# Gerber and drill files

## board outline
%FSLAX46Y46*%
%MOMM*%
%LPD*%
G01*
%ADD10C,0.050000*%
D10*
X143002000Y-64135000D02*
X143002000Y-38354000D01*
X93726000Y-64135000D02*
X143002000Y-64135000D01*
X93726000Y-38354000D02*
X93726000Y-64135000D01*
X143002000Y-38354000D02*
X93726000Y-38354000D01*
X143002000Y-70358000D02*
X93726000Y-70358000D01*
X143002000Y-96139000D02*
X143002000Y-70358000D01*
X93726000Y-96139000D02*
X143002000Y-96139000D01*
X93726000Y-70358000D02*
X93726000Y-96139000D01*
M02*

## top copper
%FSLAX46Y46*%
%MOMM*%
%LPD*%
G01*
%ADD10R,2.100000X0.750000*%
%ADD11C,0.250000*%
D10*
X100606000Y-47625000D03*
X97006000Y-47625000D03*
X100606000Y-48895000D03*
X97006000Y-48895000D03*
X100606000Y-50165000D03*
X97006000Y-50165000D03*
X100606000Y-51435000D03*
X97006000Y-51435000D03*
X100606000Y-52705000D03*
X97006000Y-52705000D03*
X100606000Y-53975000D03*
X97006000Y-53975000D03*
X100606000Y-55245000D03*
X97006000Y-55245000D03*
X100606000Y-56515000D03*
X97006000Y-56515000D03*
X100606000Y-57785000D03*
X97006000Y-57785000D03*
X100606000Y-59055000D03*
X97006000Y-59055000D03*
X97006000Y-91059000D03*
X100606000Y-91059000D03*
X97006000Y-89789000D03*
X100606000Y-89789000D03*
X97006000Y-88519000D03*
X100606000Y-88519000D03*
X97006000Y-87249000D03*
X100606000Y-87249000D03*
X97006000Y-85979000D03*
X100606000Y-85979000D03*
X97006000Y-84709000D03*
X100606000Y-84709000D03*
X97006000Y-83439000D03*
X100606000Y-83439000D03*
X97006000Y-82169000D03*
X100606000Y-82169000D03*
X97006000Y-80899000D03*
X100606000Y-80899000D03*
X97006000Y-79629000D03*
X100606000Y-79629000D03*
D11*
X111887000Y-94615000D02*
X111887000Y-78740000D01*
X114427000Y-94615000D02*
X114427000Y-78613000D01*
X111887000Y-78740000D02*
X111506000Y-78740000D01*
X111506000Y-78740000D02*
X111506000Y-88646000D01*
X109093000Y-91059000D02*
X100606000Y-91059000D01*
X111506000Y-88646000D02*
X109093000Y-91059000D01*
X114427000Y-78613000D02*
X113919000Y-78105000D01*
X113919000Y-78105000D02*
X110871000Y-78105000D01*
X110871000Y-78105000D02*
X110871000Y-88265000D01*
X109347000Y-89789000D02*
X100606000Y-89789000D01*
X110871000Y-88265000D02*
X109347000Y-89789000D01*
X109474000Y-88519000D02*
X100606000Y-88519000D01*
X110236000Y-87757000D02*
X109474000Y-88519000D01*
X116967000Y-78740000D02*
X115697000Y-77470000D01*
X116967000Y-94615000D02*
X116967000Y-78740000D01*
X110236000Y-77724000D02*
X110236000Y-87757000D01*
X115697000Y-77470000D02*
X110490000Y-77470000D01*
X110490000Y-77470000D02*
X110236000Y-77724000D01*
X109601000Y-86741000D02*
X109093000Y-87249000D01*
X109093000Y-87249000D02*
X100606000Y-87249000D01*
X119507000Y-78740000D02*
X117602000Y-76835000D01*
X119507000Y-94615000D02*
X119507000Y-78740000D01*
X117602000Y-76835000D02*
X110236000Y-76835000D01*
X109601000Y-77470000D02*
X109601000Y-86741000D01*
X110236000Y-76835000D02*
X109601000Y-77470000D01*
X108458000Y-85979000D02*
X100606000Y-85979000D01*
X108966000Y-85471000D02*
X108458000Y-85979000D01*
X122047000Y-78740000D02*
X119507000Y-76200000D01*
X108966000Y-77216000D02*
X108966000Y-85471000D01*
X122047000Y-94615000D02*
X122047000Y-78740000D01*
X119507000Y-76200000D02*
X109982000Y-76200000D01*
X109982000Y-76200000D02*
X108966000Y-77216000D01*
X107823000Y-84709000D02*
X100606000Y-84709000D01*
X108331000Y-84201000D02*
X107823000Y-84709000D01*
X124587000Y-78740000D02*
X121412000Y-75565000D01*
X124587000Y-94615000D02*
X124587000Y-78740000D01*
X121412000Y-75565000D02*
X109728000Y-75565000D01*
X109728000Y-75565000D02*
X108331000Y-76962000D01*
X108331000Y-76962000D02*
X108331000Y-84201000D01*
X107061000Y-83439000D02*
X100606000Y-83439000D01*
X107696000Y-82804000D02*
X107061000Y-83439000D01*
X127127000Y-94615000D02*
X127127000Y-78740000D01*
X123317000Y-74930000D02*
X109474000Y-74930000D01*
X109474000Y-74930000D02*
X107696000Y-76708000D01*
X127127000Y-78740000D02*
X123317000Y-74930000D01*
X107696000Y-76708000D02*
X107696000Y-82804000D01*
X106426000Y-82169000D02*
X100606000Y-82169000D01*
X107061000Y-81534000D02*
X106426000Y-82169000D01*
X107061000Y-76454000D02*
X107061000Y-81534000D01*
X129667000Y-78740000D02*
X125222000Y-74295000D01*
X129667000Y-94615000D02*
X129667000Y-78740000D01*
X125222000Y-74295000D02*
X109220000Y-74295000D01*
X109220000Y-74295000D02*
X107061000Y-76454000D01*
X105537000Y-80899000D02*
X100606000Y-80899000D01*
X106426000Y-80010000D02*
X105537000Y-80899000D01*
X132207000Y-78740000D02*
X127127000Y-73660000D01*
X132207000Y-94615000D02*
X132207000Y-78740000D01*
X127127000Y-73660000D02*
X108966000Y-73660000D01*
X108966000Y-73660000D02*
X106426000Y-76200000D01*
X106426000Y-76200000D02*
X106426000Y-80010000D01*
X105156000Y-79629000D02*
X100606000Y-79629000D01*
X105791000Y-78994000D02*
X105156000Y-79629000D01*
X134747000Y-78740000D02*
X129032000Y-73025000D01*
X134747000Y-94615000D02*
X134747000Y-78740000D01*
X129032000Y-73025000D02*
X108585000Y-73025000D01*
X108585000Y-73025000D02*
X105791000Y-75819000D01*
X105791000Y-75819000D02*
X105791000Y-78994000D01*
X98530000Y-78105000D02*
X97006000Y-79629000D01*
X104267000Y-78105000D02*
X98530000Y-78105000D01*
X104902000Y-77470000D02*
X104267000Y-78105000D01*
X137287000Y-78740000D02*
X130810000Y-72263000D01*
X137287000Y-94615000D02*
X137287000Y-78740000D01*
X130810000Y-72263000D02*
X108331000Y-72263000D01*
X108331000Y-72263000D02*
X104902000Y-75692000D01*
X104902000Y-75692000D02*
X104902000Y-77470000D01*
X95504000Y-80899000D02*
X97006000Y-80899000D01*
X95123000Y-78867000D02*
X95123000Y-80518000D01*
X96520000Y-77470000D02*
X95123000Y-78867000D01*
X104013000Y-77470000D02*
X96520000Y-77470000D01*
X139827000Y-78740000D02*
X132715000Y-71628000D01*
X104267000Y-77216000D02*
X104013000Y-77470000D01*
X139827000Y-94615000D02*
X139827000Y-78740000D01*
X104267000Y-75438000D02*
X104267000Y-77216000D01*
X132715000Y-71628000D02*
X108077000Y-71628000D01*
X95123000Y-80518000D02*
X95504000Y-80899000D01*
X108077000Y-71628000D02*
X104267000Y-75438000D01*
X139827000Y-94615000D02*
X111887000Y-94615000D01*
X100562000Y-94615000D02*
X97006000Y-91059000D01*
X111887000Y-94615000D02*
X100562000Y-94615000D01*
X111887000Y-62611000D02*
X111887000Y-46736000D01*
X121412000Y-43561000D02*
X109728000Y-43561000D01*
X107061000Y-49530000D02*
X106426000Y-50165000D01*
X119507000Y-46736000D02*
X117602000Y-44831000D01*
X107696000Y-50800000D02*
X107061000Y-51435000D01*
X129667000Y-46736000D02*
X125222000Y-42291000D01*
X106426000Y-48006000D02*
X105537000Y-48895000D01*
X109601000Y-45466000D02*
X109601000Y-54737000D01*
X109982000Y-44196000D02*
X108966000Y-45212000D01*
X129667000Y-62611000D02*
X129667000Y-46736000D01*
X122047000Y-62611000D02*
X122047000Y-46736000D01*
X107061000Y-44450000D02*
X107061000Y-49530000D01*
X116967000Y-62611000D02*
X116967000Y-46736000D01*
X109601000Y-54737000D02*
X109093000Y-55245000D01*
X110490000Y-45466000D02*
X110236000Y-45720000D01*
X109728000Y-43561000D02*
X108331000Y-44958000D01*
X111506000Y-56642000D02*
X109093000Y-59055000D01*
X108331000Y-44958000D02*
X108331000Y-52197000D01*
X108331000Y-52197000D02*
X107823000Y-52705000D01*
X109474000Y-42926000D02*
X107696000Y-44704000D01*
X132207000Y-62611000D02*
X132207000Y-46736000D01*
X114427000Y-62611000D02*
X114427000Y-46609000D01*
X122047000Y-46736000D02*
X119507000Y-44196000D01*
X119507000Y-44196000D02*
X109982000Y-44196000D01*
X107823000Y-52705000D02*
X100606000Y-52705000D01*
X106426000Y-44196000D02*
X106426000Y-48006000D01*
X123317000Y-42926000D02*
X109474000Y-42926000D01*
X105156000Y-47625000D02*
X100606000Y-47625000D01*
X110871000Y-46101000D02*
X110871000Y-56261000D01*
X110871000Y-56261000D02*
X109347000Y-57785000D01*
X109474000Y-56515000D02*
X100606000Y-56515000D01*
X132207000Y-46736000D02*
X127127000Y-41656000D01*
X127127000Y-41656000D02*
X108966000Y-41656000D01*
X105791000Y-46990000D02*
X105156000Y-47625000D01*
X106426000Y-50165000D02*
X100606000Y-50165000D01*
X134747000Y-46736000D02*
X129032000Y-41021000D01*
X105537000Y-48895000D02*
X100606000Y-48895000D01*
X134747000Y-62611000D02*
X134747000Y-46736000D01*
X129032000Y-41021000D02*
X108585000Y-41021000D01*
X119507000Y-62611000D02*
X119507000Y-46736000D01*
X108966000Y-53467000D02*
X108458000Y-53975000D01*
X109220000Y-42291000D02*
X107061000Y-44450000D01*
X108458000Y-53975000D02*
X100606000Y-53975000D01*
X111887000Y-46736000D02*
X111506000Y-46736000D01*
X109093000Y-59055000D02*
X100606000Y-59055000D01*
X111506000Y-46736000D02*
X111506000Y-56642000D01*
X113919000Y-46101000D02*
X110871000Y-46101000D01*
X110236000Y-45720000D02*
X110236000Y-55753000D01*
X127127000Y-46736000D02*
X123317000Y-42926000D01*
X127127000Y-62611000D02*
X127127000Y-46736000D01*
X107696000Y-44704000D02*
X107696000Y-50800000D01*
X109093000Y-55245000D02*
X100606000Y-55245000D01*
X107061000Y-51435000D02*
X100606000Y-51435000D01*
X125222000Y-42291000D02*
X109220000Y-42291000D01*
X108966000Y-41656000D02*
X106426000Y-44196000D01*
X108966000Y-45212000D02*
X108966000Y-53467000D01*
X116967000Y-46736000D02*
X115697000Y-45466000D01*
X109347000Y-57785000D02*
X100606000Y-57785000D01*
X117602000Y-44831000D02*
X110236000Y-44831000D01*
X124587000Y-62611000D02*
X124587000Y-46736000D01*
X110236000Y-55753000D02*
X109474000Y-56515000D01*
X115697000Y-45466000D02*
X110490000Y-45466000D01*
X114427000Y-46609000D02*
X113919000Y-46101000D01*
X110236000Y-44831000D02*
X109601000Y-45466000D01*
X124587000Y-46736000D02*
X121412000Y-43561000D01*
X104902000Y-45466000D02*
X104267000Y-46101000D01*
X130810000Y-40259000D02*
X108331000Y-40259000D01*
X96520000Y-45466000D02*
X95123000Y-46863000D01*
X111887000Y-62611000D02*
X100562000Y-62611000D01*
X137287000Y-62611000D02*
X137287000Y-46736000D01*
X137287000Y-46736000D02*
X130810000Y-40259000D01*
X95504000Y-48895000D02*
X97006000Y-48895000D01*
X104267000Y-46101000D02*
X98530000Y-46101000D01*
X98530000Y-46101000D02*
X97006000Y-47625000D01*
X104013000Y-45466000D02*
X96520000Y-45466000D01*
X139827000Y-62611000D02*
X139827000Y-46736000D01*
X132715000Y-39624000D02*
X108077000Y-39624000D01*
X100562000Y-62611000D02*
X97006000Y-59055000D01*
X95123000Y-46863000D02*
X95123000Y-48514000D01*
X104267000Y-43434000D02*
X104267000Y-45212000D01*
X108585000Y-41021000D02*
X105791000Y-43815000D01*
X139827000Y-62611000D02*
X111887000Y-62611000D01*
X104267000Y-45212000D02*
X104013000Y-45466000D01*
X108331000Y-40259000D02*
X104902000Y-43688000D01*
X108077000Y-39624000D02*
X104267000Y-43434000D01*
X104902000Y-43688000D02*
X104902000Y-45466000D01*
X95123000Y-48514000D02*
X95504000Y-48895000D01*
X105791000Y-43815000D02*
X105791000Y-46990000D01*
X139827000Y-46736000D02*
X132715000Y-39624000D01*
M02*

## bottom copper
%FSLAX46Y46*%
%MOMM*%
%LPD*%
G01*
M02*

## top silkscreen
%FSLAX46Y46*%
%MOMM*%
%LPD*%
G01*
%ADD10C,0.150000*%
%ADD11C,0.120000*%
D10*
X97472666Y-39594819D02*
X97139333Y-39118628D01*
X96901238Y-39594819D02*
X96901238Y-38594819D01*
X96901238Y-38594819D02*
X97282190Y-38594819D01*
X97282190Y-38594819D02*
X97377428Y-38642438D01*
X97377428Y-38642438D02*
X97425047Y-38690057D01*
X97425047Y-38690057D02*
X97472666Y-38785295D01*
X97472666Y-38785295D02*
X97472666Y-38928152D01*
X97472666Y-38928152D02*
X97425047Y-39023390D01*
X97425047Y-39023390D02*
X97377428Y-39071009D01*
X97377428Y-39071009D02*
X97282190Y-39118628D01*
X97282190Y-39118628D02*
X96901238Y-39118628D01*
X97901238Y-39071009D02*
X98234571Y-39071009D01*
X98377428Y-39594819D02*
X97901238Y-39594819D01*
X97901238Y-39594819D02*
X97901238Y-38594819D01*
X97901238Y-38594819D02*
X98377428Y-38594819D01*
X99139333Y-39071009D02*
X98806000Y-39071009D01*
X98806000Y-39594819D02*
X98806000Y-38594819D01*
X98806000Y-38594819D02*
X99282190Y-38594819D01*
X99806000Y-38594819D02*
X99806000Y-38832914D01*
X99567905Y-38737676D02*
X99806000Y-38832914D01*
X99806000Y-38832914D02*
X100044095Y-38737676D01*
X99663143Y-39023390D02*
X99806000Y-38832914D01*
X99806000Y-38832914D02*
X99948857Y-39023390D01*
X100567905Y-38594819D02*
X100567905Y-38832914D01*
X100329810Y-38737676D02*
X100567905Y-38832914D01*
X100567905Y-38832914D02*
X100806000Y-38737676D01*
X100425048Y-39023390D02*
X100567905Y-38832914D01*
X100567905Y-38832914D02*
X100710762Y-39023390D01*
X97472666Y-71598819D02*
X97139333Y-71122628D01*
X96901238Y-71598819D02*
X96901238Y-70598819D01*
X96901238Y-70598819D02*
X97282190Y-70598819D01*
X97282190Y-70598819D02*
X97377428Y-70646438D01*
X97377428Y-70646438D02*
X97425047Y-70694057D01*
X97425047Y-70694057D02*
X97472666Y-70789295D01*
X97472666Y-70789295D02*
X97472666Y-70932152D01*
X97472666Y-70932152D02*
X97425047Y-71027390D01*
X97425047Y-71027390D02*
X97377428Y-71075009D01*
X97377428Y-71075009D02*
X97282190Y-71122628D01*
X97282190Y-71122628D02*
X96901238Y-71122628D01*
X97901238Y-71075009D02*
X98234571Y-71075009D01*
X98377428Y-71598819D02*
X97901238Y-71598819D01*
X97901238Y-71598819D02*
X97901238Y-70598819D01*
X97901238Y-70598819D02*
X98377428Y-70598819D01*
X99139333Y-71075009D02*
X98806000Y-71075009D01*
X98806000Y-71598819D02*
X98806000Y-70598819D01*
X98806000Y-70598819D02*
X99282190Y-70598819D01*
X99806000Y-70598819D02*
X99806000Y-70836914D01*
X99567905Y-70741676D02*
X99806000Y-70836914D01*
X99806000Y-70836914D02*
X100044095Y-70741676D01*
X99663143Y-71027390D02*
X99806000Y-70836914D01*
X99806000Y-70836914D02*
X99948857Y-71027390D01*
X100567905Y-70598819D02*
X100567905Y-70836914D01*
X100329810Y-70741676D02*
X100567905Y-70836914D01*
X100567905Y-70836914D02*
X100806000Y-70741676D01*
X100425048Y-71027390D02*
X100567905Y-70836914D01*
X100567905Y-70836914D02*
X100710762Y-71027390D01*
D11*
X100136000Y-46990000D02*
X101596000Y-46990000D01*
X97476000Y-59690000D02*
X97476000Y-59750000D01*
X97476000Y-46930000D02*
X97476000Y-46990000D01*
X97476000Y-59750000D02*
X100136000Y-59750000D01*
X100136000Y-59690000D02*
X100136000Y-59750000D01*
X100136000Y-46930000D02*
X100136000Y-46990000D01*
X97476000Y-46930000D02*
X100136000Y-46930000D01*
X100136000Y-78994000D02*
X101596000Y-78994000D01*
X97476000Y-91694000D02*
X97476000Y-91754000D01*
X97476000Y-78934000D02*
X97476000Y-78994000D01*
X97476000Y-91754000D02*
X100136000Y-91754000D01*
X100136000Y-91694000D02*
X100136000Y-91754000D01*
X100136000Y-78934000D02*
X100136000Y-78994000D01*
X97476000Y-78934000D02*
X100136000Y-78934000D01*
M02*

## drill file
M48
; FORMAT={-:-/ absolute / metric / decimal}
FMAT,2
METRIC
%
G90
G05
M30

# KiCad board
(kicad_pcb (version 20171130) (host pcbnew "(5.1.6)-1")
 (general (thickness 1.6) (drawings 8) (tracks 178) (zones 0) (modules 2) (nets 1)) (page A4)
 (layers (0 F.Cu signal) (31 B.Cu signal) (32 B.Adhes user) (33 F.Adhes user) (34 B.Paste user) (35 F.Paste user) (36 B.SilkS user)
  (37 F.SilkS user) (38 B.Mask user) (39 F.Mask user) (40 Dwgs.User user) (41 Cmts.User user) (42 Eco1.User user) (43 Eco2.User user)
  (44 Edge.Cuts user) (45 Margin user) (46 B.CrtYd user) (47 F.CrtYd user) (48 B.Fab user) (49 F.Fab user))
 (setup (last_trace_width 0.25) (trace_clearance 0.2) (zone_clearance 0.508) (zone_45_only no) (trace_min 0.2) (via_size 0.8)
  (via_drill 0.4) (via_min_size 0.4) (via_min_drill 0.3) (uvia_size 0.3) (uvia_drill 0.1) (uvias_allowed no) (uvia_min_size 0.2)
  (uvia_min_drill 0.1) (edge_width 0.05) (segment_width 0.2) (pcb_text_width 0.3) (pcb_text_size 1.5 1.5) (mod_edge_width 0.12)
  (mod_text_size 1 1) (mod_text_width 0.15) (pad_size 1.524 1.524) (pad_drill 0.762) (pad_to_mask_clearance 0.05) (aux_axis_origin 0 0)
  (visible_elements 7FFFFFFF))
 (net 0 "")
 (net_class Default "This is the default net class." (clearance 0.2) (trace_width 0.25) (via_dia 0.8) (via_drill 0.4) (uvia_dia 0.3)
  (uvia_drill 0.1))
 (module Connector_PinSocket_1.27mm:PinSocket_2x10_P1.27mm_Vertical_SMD (layer F.Cu) (at 98.806 53.34)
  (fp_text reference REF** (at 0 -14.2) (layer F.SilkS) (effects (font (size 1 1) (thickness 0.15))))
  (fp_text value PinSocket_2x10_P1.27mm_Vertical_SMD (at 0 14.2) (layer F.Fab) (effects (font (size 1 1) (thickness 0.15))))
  (fp_line (start 1.33 -6.35) (end 2.79 -6.35) (layer F.SilkS) (width 0.12))
  (fp_line (start -1.33 6.35) (end -1.33 6.41) (layer F.SilkS) (width 0.12))
  (fp_line (start -1.33 -6.41) (end -1.33 -6.35) (layer F.SilkS) (width 0.12))
  (fp_line (start -1.33 6.41) (end 1.33 6.41) (layer F.SilkS) (width 0.12))
  (fp_line (start 1.33 6.35) (end 1.33 6.41) (layer F.SilkS) (width 0.12))
  (fp_line (start 1.33 -6.41) (end 1.33 -6.35) (layer F.SilkS) (width 0.12))
  (fp_line (start -1.33 -6.41) (end 1.33 -6.41) (layer F.SilkS) (width 0.12))
  (pad 1 smd rect (at 1.8 -5.715) (size 2.1 0.75) (layers F.Cu F.Paste F.Mask))
  (pad 2 smd rect (at -1.8 -5.715) (size 2.1 0.75) (layers F.Cu F.Paste F.Mask))
  (pad 3 smd rect (at 1.8 -4.445) (size 2.1 0.75) (layers F.Cu F.Paste F.Mask))
  (pad 4 smd rect (at -1.8 -4.445) (size 2.1 0.75) (layers F.Cu F.Paste F.Mask))
  (pad 5 smd rect (at 1.8 -3.175) (size 2.1 0.75) (layers F.Cu F.Paste F.Mask))
  (pad 6 smd rect (at -1.8 -3.175) (size 2.1 0.75) (layers F.Cu F.Paste F.Mask))
  (pad 7 smd rect (at 1.8 -1.905) (size 2.1 0.75) (layers F.Cu F.Paste F.Mask))
  (pad 8 smd rect (at -1.8 -1.905) (size 2.1 0.75) (layers F.Cu F.Paste F.Mask))
  (pad 9 smd rect (at 1.8 -0.635) (size 2.1 0.75) (layers F.Cu F.Paste F.Mask))
  (pad 10 smd rect (at -1.8 -0.635) (size 2.1 0.75) (layers F.Cu F.Paste F.Mask))
  (pad 11 smd rect (at 1.8 0.635) (size 2.1 0.75) (layers F.Cu F.Paste F.Mask))
  (pad 12 smd rect (at -1.8 0.635) (size 2.1 0.75) (layers F.Cu F.Paste F.Mask))
  (pad 13 smd rect (at 1.8 1.905) (size 2.1 0.75) (layers F.Cu F.Paste F.Mask))
  (pad 14 smd rect (at -1.8 1.905) (size 2.1 0.75) (layers F.Cu F.Paste F.Mask))
  (pad 15 smd rect (at 1.8 3.175) (size 2.1 0.75) (layers F.Cu F.Paste F.Mask))
  (pad 16 smd rect (at -1.8 3.175) (size 2.1 0.75) (layers F.Cu F.Paste F.Mask))
  (pad 17 smd rect (at 1.8 4.445) (size 2.1 0.75) (layers F.Cu F.Paste F.Mask))
  (pad 18 smd rect (at -1.8 4.445) (size 2.1 0.75) (layers F.Cu F.Paste F.Mask))
  (pad 19 smd rect (at 1.8 5.715) (size 2.1 0.75) (layers F.Cu F.Paste F.Mask))
  (pad 20 smd rect (at -1.8 5.715) (size 2.1 0.75) (layers F.Cu F.Paste F.Mask)))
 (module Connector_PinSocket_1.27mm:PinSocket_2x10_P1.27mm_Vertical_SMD (layer F.Cu) (at 98.806 85.344)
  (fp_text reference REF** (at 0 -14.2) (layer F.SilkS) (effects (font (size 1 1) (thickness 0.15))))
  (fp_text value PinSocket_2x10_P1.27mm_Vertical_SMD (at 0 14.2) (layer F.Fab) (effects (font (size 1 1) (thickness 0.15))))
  (fp_line (start 1.33 -6.35) (end 2.79 -6.35) (layer F.SilkS) (width 0.12))
  (fp_line (start -1.33 6.35) (end -1.33 6.41) (layer F.SilkS) (width 0.12))
  (fp_line (start -1.33 -6.41) (end -1.33 -6.35) (layer F.SilkS) (width 0.12))
  (fp_line (start -1.33 6.41) (end 1.33 6.41) (layer F.SilkS) (width 0.12))
  (fp_line (start 1.33 6.35) (end 1.33 6.41) (layer F.SilkS) (width 0.12))
  (fp_line (start 1.33 -6.41) (end 1.33 -6.35) (layer F.SilkS) (width 0.12))
  (fp_line (start -1.33 -6.41) (end 1.33 -6.41) (layer F.SilkS) (width 0.12))
  (pad 20 smd rect (at -1.8 5.715) (size 2.1 0.75) (layers F.Cu F.Paste F.Mask))
  (pad 19 smd rect (at 1.8 5.715) (size 2.1 0.75) (layers F.Cu F.Paste F.Mask))
  (pad 18 smd rect (at -1.8 4.445) (size 2.1 0.75) (layers F.Cu F.Paste F.Mask))
  (pad 17 smd rect (at 1.8 4.445) (size 2.1 0.75) (layers F.Cu F.Paste F.Mask))
  (pad 16 smd rect (at -1.8 3.175) (size 2.1 0.75) (layers F.Cu F.Paste F.Mask))
  (pad 15 smd rect (at 1.8 3.175) (size 2.1 0.75) (layers F.Cu F.Paste F.Mask))
  (pad 14 smd rect (at -1.8 1.905) (size 2.1 0.75) (layers F.Cu F.Paste F.Mask))
  (pad 13 smd rect (at 1.8 1.905) (size 2.1 0.75) (layers F.Cu F.Paste F.Mask))
  (pad 12 smd rect (at -1.8 0.635) (size 2.1 0.75) (layers F.Cu F.Paste F.Mask))
  (pad 11 smd rect (at 1.8 0.635) (size 2.1 0.75) (layers F.Cu F.Paste F.Mask))
  (pad 10 smd rect (at -1.8 -0.635) (size 2.1 0.75) (layers F.Cu F.Paste F.Mask))
  (pad 9 smd rect (at 1.8 -0.635) (size 2.1 0.75) (layers F.Cu F.Paste F.Mask))
  (pad 8 smd rect (at -1.8 -1.905) (size 2.1 0.75) (layers F.Cu F.Paste F.Mask))
  (pad 7 smd rect (at 1.8 -1.905) (size 2.1 0.75) (layers F.Cu F.Paste F.Mask))
  (pad 6 smd rect (at -1.8 -3.175) (size 2.1 0.75) (layers F.Cu F.Paste F.Mask))
  (pad 5 smd rect (at 1.8 -3.175) (size 2.1 0.75) (layers F.Cu F.Paste F.Mask))
  (pad 4 smd rect (at -1.8 -4.445) (size 2.1 0.75) (layers F.Cu F.Paste F.Mask))
  (pad 3 smd rect (at 1.8 -4.445) (size 2.1 0.75) (layers F.Cu F.Paste F.Mask))
  (pad 2 smd rect (at -1.8 -5.715) (size 2.1 0.75) (layers F.Cu F.Paste F.Mask))
  (pad 1 smd rect (at 1.8 -5.715) (size 2.1 0.75) (layers F.Cu F.Paste F.Mask)))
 (gr_line (start 143.002 64.135) (end 143.002 38.354) (layer Edge.Cuts) (width 0.05))
 (gr_line (start 93.726 64.135) (end 143.002 64.135) (layer Edge.Cuts) (width 0.05))
 (gr_line (start 93.726 38.354) (end 93.726 64.135) (layer Edge.Cuts) (width 0.05))
 (gr_line (start 143.002 38.354) (end 93.726 38.354) (layer Edge.Cuts) (width 0.05))
 (gr_line (start 143.002 70.358) (end 93.726 70.358) (layer Edge.Cuts) (width 0.05))
 (gr_line (start 143.002 96.139) (end 143.002 70.358) (layer Edge.Cuts) (width 0.05))
 (gr_line (start 93.726 96.139) (end 143.002 96.139) (layer Edge.Cuts) (width 0.05))
 (gr_line (start 93.726 70.358) (end 93.726 96.139) (layer Edge.Cuts) (width 0.05))
 (segment (start 111.887 94.615) (end 111.887 78.74) (width 0.25) (layer F.Cu) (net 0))
 (segment (start 114.427 94.615) (end 114.427 78.613) (width 0.25) (layer F.Cu) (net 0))
 (segment (start 111.887 78.74) (end 111.506 78.74) (width 0.25) (layer F.Cu) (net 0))
 (segment (start 111.506 78.74) (end 111.506 88.646) (width 0.25) (layer F.Cu) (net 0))
 (segment (start 109.093 91.059) (end 100.606 91.059) (width 0.25) (layer F.Cu) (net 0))
 (segment (start 111.506 88.646) (end 109.093 91.059) (width 0.25) (layer F.Cu) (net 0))
 (segment (start 114.427 78.613) (end 113.919 78.105) (width 0.25) (layer F.Cu) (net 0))
 (segment (start 113.919 78.105) (end 110.871 78.105) (width 0.25) (layer F.Cu) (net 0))
 (segment (start 110.871 78.105) (end 110.871 88.265) (width 0.25) (layer F.Cu) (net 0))
 (segment (start 109.347 89.789) (end 100.606 89.789) (width 0.25) (layer F.Cu) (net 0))
 (segment (start 110.871 88.265) (end 109.347 89.789) (width 0.25) (layer F.Cu) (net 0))
 (segment (start 109.474 88.519) (end 100.606 88.519) (width 0.25) (layer F.Cu) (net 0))
 (segment (start 110.236 87.757) (end 109.474 88.519) (width 0.25) (layer F.Cu) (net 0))
 (segment (start 116.967 78.74) (end 115.697 77.47) (width 0.25) (layer F.Cu) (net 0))
 (segment (start 116.967 94.615) (end 116.967 78.74) (width 0.25) (layer F.Cu) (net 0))
 (segment (start 110.236 77.724) (end 110.236 87.757) (width 0.25) (layer F.Cu) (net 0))
 (segment (start 115.697 77.47) (end 110.49 77.47) (width 0.25) (layer F.Cu) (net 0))
 (segment (start 110.49 77.47) (end 110.236 77.724) (width 0.25) (layer F.Cu) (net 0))
 (segment (start 109.601 86.741) (end 109.093 87.249) (width 0.25) (layer F.Cu) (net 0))
 (segment (start 109.093 87.249) (end 100.606 87.249) (width 0.25) (layer F.Cu) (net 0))
 (segment (start 119.507 78.74) (end 117.602 76.835) (width 0.25) (layer F.Cu) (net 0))
 (segment (start 119.507 94.615) (end 119.507 78.74) (width 0.25) (layer F.Cu) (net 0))
 (segment (start 117.602 76.835) (end 110.236 76.835) (width 0.25) (layer F.Cu) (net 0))
 (segment (start 109.601 77.47) (end 109.601 86.741) (width 0.25) (layer F.Cu) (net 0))
 (segment (start 110.236 76.835) (end 109.601 77.47) (width 0.25) (layer F.Cu) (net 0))
 (segment (start 108.458 85.979) (end 100.606 85.979) (width 0.25) (layer F.Cu) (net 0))
 (segment (start 108.966 85.471) (end 108.458 85.979) (width 0.25) (layer F.Cu) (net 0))
 (segment (start 122.047 78.74) (end 119.507 76.2) (width 0.25) (layer F.Cu) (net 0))
 (segment (start 108.966 77.216) (end 108.966 85.471) (width 0.25) (layer F.Cu) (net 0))
 (segment (start 122.047 94.615) (end 122.047 78.74) (width 0.25) (layer F.Cu) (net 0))
 (segment (start 119.507 76.2) (end 109.982 76.2) (width 0.25) (layer F.Cu) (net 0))
 (segment (start 109.982 76.2) (end 108.966 77.216) (width 0.25) (layer F.Cu) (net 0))
 (segment (start 107.823 84.709) (end 100.606 84.709) (width 0.25) (layer F.Cu) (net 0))
 (segment (start 108.331 84.201) (end 107.823 84.709) (width 0.25) (layer F.Cu) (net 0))
 (segment (start 124.587 78.74) (end 121.412 75.565) (width 0.25) (layer F.Cu) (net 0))
 (segment (start 124.587 94.615) (end 124.587 78.74) (width 0.25) (layer F.Cu) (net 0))
 (segment (start 121.412 75.565) (end 109.728 75.565) (width 0.25) (layer F.Cu) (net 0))
 (segment (start 109.728 75.565) (end 108.331 76.962) (width 0.25) (layer F.Cu) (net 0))
 (segment (start 108.331 76.962) (end 108.331 84.201) (width 0.25) (layer F.Cu) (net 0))
 (segment (start 107.061 83.439) (end 100.606 83.439) (width 0.25) (layer F.Cu) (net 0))
 (segment (start 107.696 82.804) (end 107.061 83.439) (width 0.25) (layer F.Cu) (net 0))
 (segment (start 127.127 94.615) (end 127.127 78.74) (width 0.25) (layer F.Cu) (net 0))
 (segment (start 123.317 74.93) (end 109.474 74.93) (width 0.25) (layer F.Cu) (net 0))
 (segment (start 109.474 74.93) (end 107.696 76.708) (width 0.25) (layer F.Cu) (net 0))
 (segment (start 127.127 78.74) (end 123.317 74.93) (width 0.25) (layer F.Cu) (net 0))
 (segment (start 107.696 76.708) (end 107.696 82.804) (width 0.25) (layer F.Cu) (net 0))
 (segment (start 106.426 82.169) (end 100.606 82.169) (width 0.25) (layer F.Cu) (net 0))
 (segment (start 107.061 81.534) (end 106.426 82.169) (width 0.25) (layer F.Cu) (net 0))
 (segment (start 107.061 76.454) (end 107.061 81.534) (width 0.25) (layer F.Cu) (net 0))
 (segment (start 129.667 78.74) (end 125.222 74.295) (width 0.25) (layer F.Cu) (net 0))
 (segment (start 129.667 94.615) (end 129.667 78.74) (width 0.25) (layer F.Cu) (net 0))
 (segment (start 125.222 74.295) (end 109.22 74.295) (width 0.25) (layer F.Cu) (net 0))
 (segment (start 109.22 74.295) (end 107.061 76.454) (width 0.25) (layer F.Cu) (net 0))
 (segment (start 105.537 80.899) (end 100.606 80.899) (width 0.25) (layer F.Cu) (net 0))
 (segment (start 106.426 80.01) (end 105.537 80.899) (width 0.25) (layer F.Cu) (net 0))
 (segment (start 132.207 78.74) (end 127.127 73.66) (width 0.25) (layer F.Cu) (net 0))
 (segment (start 132.207 94.615) (end 132.207 78.74) (width 0.25) (layer F.Cu) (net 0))
 (segment (start 127.127 73.66) (end 108.966 73.66) (width 0.25) (layer F.Cu) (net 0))
 (segment (start 108.966 73.66) (end 106.426 76.2) (width 0.25) (layer F.Cu) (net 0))
 (segment (start 106.426 76.2) (end 106.426 80.01) (width 0.25) (layer F.Cu) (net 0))
 (segment (start 105.156 79.629) (end 100.606 79.629) (width 0.25) (layer F.Cu) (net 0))
 (segment (start 105.791 78.994) (end 105.156 79.629) (width 0.25) (layer F.Cu) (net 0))
 (segment (start 134.747 78.74) (end 129.032 73.025) (width 0.25) (layer F.Cu) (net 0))
 (segment (start 134.747 94.615) (end 134.747 78.74) (width 0.25) (layer F.Cu) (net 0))
 (segment (start 129.032 73.025) (end 108.585 73.025) (width 0.25) (layer F.Cu) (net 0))
 (segment (start 108.585 73.025) (end 105.791 75.819) (width 0.25) (layer F.Cu) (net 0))
 (segment (start 105.791 75.819) (end 105.791 78.994) (width 0.25) (layer F.Cu) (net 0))
 (segment (start 98.53 78.105) (end 97.006 79.629) (width 0.25) (layer F.Cu) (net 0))
 (segment (start 104.267 78.105) (end 98.53 78.105) (width 0.25) (layer F.Cu) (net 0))
 (segment (start 104.902 77.47) (end 104.267 78.105) (width 0.25) (layer F.Cu) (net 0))
 (segment (start 137.287 78.74) (end 130.81 72.263) (width 0.25) (layer F.Cu) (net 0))
 (segment (start 137.287 94.615) (end 137.287 78.74) (width 0.25) (layer F.Cu) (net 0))
 (segment (start 130.81 72.263) (end 108.331 72.263) (width 0.25) (layer F.Cu) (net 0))
 (segment (start 108.331 72.263) (end 104.902 75.692) (width 0.25) (layer F.Cu) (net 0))
 (segment (start 104.902 75.692) (end 104.902 77.47) (width 0.25) (layer F.Cu) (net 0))
 (segment (start 95.504 80.899) (end 97.006 80.899) (width 0.25) (layer F.Cu) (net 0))
 (segment (start 95.123 78.867) (end 95.123 80.518) (width 0.25) (layer F.Cu) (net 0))
 (segment (start 96.52 77.47) (end 95.123 78.867) (width 0.25) (layer F.Cu) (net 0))
 (segment (start 104.013 77.47) (end 96.52 77.47) (width 0.25) (layer F.Cu) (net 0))
 (segment (start 139.827 78.74) (end 132.715 71.628) (width 0.25) (layer F.Cu) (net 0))
 (segment (start 104.267 77.216) (end 104.013 77.47) (width 0.25) (layer F.Cu) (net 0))
 (segment (start 139.827 94.615) (end 139.827 78.74) (width 0.25) (layer F.Cu) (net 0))
 (segment (start 104.267 75.438) (end 104.267 77.216) (width 0.25) (layer F.Cu) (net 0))
 (segment (start 132.715 71.628) (end 108.077 71.628) (width 0.25) (layer F.Cu) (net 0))
 (segment (start 95.123 80.518) (end 95.504 80.899) (width 0.25) (layer F.Cu) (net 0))
 (segment (start 108.077 71.628) (end 104.267 75.438) (width 0.25) (layer F.Cu) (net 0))
 (segment (start 139.827 94.615) (end 111.887 94.615) (width 0.25) (layer F.Cu) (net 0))
 (segment (start 100.562 94.615) (end 97.006 91.059) (width 0.25) (layer F.Cu) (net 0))
 (segment (start 111.887 94.615) (end 100.562 94.615) (width 0.25) (layer F.Cu) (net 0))
 (segment (start 111.887 62.611) (end 111.887 46.736) (width 0.25) (layer F.Cu) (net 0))
 (segment (start 121.412 43.561) (end 109.728 43.561) (width 0.25) (layer F.Cu) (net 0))
 (segment (start 107.061 49.53) (end 106.426 50.165) (width 0.25) (layer F.Cu) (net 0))
 (segment (start 119.507 46.736) (end 117.602 44.831) (width 0.25) (layer F.Cu) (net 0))
 (segment (start 107.696 50.8) (end 107.061 51.435) (width 0.25) (layer F.Cu) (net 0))
 (segment (start 129.667 46.736) (end 125.222 42.291) (width 0.25) (layer F.Cu) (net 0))
 (segment (start 106.426 48.006) (end 105.537 48.895) (width 0.25) (layer F.Cu) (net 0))
 (segment (start 109.601 45.466) (end 109.601 54.737) (width 0.25) (layer F.Cu) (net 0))
 (segment (start 109.982 44.196) (end 108.966 45.212) (width 0.25) (layer F.Cu) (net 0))
 (segment (start 129.667 62.611) (end 129.667 46.736) (width 0.25) (layer F.Cu) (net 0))
 (segment (start 122.047 62.611) (end 122.047 46.736) (width 0.25) (layer F.Cu) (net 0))
 (segment (start 107.061 44.45) (end 107.061 49.53) (width 0.25) (layer F.Cu) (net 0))
 (segment (start 116.967 62.611) (end 116.967 46.736) (width 0.25) (layer F.Cu) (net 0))
 (segment (start 109.601 54.737) (end 109.093 55.245) (width 0.25) (layer F.Cu) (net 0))
 (segment (start 110.49 45.466) (end 110.236 45.72) (width 0.25) (layer F.Cu) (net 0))
 (segment (start 109.728 43.561) (end 108.331 44.958) (width 0.25) (layer F.Cu) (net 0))
 (segment (start 111.506 56.642) (end 109.093 59.055) (width 0.25) (layer F.Cu) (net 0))
 (segment (start 108.331 44.958) (end 108.331 52.197) (width 0.25) (layer F.Cu) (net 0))
 (segment (start 108.331 52.197) (end 107.823 52.705) (width 0.25) (layer F.Cu) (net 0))
 (segment (start 109.474 42.926) (end 107.696 44.704) (width 0.25) (layer F.Cu) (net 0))
 (segment (start 132.207 62.611) (end 132.207 46.736) (width 0.25) (layer F.Cu) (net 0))
 (segment (start 114.427 62.611) (end 114.427 46.609) (width 0.25) (layer F.Cu) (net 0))
 (segment (start 122.047 46.736) (end 119.507 44.196) (width 0.25) (layer F.Cu) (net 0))
 (segment (start 119.507 44.196) (end 109.982 44.196) (width 0.25) (layer F.Cu) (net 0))
 (segment (start 107.823 52.705) (end 100.606 52.705) (width 0.25) (layer F.Cu) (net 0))
 (segment (start 106.426 44.196) (end 106.426 48.006) (width 0.25) (layer F.Cu) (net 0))
 (segment (start 123.317 42.926) (end 109.474 42.926) (width 0.25) (layer F.Cu) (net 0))
 (segment (start 105.156 47.625) (end 100.606 47.625) (width 0.25) (layer F.Cu) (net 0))
 (segment (start 110.871 46.101) (end 110.871 56.261) (width 0.25) (layer F.Cu) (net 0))
 (segment (start 110.871 56.261) (end 109.347 57.785) (width 0.25) (layer F.Cu) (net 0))
 (segment (start 109.474 56.515) (end 100.606 56.515) (width 0.25) (layer F.Cu) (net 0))
 (segment (start 132.207 46.736) (end 127.127 41.656) (width 0.25) (layer F.Cu) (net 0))
 (segment (start 127.127 41.656) (end 108.966 41.656) (width 0.25) (layer F.Cu) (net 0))
 (segment (start 105.791 46.99) (end 105.156 47.625) (width 0.25) (layer F.Cu) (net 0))
 (segment (start 106.426 50.165) (end 100.606 50.165) (width 0.25) (layer F.Cu) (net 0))
 (segment (start 134.747 46.736) (end 129.032 41.021) (width 0.25) (layer F.Cu) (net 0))
 (segment (start 105.537 48.895) (end 100.606 48.895) (width 0.25) (layer F.Cu) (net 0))
 (segment (start 134.747 62.611) (end 134.747 46.736) (width 0.25) (layer F.Cu) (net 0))
 (segment (start 129.032 41.021) (end 108.585 41.021) (width 0.25) (layer F.Cu) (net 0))
 (segment (start 119.507 62.611) (end 119.507 46.736) (width 0.25) (layer F.Cu) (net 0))
 (segment (start 108.966 53.467) (end 108.458 53.975) (width 0.25) (layer F.Cu) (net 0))
 (segment (start 109.22 42.291) (end 107.061 44.45) (width 0.25) (layer F.Cu) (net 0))
 (segment (start 108.458 53.975) (end 100.606 53.975) (width 0.25) (layer F.Cu) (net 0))
 (segment (start 111.887 46.736) (end 111.506 46.736) (width 0.25) (layer F.Cu) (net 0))
 (segment (start 109.093 59.055) (end 100.606 59.055) (width 0.25) (layer F.Cu) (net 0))
 (segment (start 111.506 46.736) (end 111.506 56.642) (width 0.25) (layer F.Cu) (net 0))
 (segment (start 113.919 46.101) (end 110.871 46.101) (width 0.25) (layer F.Cu) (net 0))
 (segment (start 110.236 45.72) (end 110.236 55.753) (width 0.25) (layer F.Cu) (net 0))
 (segment (start 127.127 46.736) (end 123.317 42.926) (width 0.25) (layer F.Cu) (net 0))
 (segment (start 127.127 62.611) (end 127.127 46.736) (width 0.25) (layer F.Cu) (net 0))
 (segment (start 107.696 44.704) (end 107.696 50.8) (width 0.25) (layer F.Cu) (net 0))
 (segment (start 109.093 55.245) (end 100.606 55.245) (width 0.25) (layer F.Cu) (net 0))
 (segment (start 107.061 51.435) (end 100.606 51.435) (width 0.25) (layer F.Cu) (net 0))
 (segment (start 125.222 42.291) (end 109.22 42.291) (width 0.25) (layer F.Cu) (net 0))
 (segment (start 108.966 41.656) (end 106.426 44.196) (width 0.25) (layer F.Cu) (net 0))
 (segment (start 108.966 45.212) (end 108.966 53.467) (width 0.25) (layer F.Cu) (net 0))
 (segment (start 116.967 46.736) (end 115.697 45.466) (width 0.25) (layer F.Cu) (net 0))
 (segment (start 109.347 57.785) (end 100.606 57.785) (width 0.25) (layer F.Cu) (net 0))
 (segment (start 117.602 44.831) (end 110.236 44.831) (width 0.25) (layer F.Cu) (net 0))
 (segment (start 124.587 62.611) (end 124.587 46.736) (width 0.25) (layer F.Cu) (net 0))
 (segment (start 110.236 55.753) (end 109.474 56.515) (width 0.25) (layer F.Cu) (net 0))
 (segment (start 115.697 45.466) (end 110.49 45.466) (width 0.25) (layer F.Cu) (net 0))
 (segment (start 114.427 46.609) (end 113.919 46.101) (width 0.25) (layer F.Cu) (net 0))
 (segment (start 110.236 44.831) (end 109.601 45.466) (width 0.25) (layer F.Cu) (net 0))
 (segment (start 124.587 46.736) (end 121.412 43.561) (width 0.25) (layer F.Cu) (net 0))
 (segment (start 104.902 45.466) (end 104.267 46.101) (width 0.25) (layer F.Cu) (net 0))
 (segment (start 130.81 40.259) (end 108.331 40.259) (width 0.25) (layer F.Cu) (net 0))
 (segment (start 96.52 45.466) (end 95.123 46.863) (width 0.25) (layer F.Cu) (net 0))
 (segment (start 111.887 62.611) (end 100.562 62.611) (width 0.25) (layer F.Cu) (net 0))
 (segment (start 137.287 62.611) (end 137.287 46.736) (width 0.25) (layer F.Cu) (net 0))
 (segment (start 137.287 46.736) (end 130.81 40.259) (width 0.25) (layer F.Cu) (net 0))
 (segment (start 95.504 48.895) (end 97.006 48.895) (width 0.25) (layer F.Cu) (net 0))
 (segment (start 104.267 46.101) (end 98.53 46.101) (width 0.25) (layer F.Cu) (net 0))
 (segment (start 98.53 46.101) (end 97.006 47.625) (width 0.25) (layer F.Cu) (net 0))
 (segment (start 104.013 45.466) (end 96.52 45.466) (width 0.25) (layer F.Cu) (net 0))
 (segment (start 139.827 62.611) (end 139.827 46.736) (width 0.25) (layer F.Cu) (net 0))
 (segment (start 132.715 39.624) (end 108.077 39.624) (width 0.25) (layer F.Cu) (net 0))
 (segment (start 100.562 62.611) (end 97.006 59.055) (width 0.25) (layer F.Cu) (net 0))
 (segment (start 95.123 46.863) (end 95.123 48.514) (width 0.25) (layer F.Cu) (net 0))
 (segment (start 104.267 43.434) (end 104.267 45.212) (width 0.25) (layer F.Cu) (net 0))
 (segment (start 108.585 41.021) (end 105.791 43.815) (width 0.25) (layer F.Cu) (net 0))
 (segment (start 139.827 62.611) (end 111.887 62.611) (width 0.25) (layer F.Cu) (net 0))
 (segment (start 104.267 45.212) (end 104.013 45.466) (width 0.25) (layer F.Cu) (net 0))
 (segment (start 108.331 40.259) (end 104.902 43.688) (width 0.25) (layer F.Cu) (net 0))
 (segment (start 108.077 39.624) (end 104.267 43.434) (width 0.25) (layer F.Cu) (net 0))
 (segment (start 104.902 43.688) (end 104.902 45.466) (width 0.25) (layer F.Cu) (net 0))
 (segment (start 95.123 48.514) (end 95.504 48.895) (width 0.25) (layer F.Cu) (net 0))
 (segment (start 105.791 43.815) (end 105.791 46.99) (width 0.25) (layer F.Cu) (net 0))
 (segment (start 139.827 46.736) (end 132.715 39.624) (width 0.25) (layer F.Cu) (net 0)))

